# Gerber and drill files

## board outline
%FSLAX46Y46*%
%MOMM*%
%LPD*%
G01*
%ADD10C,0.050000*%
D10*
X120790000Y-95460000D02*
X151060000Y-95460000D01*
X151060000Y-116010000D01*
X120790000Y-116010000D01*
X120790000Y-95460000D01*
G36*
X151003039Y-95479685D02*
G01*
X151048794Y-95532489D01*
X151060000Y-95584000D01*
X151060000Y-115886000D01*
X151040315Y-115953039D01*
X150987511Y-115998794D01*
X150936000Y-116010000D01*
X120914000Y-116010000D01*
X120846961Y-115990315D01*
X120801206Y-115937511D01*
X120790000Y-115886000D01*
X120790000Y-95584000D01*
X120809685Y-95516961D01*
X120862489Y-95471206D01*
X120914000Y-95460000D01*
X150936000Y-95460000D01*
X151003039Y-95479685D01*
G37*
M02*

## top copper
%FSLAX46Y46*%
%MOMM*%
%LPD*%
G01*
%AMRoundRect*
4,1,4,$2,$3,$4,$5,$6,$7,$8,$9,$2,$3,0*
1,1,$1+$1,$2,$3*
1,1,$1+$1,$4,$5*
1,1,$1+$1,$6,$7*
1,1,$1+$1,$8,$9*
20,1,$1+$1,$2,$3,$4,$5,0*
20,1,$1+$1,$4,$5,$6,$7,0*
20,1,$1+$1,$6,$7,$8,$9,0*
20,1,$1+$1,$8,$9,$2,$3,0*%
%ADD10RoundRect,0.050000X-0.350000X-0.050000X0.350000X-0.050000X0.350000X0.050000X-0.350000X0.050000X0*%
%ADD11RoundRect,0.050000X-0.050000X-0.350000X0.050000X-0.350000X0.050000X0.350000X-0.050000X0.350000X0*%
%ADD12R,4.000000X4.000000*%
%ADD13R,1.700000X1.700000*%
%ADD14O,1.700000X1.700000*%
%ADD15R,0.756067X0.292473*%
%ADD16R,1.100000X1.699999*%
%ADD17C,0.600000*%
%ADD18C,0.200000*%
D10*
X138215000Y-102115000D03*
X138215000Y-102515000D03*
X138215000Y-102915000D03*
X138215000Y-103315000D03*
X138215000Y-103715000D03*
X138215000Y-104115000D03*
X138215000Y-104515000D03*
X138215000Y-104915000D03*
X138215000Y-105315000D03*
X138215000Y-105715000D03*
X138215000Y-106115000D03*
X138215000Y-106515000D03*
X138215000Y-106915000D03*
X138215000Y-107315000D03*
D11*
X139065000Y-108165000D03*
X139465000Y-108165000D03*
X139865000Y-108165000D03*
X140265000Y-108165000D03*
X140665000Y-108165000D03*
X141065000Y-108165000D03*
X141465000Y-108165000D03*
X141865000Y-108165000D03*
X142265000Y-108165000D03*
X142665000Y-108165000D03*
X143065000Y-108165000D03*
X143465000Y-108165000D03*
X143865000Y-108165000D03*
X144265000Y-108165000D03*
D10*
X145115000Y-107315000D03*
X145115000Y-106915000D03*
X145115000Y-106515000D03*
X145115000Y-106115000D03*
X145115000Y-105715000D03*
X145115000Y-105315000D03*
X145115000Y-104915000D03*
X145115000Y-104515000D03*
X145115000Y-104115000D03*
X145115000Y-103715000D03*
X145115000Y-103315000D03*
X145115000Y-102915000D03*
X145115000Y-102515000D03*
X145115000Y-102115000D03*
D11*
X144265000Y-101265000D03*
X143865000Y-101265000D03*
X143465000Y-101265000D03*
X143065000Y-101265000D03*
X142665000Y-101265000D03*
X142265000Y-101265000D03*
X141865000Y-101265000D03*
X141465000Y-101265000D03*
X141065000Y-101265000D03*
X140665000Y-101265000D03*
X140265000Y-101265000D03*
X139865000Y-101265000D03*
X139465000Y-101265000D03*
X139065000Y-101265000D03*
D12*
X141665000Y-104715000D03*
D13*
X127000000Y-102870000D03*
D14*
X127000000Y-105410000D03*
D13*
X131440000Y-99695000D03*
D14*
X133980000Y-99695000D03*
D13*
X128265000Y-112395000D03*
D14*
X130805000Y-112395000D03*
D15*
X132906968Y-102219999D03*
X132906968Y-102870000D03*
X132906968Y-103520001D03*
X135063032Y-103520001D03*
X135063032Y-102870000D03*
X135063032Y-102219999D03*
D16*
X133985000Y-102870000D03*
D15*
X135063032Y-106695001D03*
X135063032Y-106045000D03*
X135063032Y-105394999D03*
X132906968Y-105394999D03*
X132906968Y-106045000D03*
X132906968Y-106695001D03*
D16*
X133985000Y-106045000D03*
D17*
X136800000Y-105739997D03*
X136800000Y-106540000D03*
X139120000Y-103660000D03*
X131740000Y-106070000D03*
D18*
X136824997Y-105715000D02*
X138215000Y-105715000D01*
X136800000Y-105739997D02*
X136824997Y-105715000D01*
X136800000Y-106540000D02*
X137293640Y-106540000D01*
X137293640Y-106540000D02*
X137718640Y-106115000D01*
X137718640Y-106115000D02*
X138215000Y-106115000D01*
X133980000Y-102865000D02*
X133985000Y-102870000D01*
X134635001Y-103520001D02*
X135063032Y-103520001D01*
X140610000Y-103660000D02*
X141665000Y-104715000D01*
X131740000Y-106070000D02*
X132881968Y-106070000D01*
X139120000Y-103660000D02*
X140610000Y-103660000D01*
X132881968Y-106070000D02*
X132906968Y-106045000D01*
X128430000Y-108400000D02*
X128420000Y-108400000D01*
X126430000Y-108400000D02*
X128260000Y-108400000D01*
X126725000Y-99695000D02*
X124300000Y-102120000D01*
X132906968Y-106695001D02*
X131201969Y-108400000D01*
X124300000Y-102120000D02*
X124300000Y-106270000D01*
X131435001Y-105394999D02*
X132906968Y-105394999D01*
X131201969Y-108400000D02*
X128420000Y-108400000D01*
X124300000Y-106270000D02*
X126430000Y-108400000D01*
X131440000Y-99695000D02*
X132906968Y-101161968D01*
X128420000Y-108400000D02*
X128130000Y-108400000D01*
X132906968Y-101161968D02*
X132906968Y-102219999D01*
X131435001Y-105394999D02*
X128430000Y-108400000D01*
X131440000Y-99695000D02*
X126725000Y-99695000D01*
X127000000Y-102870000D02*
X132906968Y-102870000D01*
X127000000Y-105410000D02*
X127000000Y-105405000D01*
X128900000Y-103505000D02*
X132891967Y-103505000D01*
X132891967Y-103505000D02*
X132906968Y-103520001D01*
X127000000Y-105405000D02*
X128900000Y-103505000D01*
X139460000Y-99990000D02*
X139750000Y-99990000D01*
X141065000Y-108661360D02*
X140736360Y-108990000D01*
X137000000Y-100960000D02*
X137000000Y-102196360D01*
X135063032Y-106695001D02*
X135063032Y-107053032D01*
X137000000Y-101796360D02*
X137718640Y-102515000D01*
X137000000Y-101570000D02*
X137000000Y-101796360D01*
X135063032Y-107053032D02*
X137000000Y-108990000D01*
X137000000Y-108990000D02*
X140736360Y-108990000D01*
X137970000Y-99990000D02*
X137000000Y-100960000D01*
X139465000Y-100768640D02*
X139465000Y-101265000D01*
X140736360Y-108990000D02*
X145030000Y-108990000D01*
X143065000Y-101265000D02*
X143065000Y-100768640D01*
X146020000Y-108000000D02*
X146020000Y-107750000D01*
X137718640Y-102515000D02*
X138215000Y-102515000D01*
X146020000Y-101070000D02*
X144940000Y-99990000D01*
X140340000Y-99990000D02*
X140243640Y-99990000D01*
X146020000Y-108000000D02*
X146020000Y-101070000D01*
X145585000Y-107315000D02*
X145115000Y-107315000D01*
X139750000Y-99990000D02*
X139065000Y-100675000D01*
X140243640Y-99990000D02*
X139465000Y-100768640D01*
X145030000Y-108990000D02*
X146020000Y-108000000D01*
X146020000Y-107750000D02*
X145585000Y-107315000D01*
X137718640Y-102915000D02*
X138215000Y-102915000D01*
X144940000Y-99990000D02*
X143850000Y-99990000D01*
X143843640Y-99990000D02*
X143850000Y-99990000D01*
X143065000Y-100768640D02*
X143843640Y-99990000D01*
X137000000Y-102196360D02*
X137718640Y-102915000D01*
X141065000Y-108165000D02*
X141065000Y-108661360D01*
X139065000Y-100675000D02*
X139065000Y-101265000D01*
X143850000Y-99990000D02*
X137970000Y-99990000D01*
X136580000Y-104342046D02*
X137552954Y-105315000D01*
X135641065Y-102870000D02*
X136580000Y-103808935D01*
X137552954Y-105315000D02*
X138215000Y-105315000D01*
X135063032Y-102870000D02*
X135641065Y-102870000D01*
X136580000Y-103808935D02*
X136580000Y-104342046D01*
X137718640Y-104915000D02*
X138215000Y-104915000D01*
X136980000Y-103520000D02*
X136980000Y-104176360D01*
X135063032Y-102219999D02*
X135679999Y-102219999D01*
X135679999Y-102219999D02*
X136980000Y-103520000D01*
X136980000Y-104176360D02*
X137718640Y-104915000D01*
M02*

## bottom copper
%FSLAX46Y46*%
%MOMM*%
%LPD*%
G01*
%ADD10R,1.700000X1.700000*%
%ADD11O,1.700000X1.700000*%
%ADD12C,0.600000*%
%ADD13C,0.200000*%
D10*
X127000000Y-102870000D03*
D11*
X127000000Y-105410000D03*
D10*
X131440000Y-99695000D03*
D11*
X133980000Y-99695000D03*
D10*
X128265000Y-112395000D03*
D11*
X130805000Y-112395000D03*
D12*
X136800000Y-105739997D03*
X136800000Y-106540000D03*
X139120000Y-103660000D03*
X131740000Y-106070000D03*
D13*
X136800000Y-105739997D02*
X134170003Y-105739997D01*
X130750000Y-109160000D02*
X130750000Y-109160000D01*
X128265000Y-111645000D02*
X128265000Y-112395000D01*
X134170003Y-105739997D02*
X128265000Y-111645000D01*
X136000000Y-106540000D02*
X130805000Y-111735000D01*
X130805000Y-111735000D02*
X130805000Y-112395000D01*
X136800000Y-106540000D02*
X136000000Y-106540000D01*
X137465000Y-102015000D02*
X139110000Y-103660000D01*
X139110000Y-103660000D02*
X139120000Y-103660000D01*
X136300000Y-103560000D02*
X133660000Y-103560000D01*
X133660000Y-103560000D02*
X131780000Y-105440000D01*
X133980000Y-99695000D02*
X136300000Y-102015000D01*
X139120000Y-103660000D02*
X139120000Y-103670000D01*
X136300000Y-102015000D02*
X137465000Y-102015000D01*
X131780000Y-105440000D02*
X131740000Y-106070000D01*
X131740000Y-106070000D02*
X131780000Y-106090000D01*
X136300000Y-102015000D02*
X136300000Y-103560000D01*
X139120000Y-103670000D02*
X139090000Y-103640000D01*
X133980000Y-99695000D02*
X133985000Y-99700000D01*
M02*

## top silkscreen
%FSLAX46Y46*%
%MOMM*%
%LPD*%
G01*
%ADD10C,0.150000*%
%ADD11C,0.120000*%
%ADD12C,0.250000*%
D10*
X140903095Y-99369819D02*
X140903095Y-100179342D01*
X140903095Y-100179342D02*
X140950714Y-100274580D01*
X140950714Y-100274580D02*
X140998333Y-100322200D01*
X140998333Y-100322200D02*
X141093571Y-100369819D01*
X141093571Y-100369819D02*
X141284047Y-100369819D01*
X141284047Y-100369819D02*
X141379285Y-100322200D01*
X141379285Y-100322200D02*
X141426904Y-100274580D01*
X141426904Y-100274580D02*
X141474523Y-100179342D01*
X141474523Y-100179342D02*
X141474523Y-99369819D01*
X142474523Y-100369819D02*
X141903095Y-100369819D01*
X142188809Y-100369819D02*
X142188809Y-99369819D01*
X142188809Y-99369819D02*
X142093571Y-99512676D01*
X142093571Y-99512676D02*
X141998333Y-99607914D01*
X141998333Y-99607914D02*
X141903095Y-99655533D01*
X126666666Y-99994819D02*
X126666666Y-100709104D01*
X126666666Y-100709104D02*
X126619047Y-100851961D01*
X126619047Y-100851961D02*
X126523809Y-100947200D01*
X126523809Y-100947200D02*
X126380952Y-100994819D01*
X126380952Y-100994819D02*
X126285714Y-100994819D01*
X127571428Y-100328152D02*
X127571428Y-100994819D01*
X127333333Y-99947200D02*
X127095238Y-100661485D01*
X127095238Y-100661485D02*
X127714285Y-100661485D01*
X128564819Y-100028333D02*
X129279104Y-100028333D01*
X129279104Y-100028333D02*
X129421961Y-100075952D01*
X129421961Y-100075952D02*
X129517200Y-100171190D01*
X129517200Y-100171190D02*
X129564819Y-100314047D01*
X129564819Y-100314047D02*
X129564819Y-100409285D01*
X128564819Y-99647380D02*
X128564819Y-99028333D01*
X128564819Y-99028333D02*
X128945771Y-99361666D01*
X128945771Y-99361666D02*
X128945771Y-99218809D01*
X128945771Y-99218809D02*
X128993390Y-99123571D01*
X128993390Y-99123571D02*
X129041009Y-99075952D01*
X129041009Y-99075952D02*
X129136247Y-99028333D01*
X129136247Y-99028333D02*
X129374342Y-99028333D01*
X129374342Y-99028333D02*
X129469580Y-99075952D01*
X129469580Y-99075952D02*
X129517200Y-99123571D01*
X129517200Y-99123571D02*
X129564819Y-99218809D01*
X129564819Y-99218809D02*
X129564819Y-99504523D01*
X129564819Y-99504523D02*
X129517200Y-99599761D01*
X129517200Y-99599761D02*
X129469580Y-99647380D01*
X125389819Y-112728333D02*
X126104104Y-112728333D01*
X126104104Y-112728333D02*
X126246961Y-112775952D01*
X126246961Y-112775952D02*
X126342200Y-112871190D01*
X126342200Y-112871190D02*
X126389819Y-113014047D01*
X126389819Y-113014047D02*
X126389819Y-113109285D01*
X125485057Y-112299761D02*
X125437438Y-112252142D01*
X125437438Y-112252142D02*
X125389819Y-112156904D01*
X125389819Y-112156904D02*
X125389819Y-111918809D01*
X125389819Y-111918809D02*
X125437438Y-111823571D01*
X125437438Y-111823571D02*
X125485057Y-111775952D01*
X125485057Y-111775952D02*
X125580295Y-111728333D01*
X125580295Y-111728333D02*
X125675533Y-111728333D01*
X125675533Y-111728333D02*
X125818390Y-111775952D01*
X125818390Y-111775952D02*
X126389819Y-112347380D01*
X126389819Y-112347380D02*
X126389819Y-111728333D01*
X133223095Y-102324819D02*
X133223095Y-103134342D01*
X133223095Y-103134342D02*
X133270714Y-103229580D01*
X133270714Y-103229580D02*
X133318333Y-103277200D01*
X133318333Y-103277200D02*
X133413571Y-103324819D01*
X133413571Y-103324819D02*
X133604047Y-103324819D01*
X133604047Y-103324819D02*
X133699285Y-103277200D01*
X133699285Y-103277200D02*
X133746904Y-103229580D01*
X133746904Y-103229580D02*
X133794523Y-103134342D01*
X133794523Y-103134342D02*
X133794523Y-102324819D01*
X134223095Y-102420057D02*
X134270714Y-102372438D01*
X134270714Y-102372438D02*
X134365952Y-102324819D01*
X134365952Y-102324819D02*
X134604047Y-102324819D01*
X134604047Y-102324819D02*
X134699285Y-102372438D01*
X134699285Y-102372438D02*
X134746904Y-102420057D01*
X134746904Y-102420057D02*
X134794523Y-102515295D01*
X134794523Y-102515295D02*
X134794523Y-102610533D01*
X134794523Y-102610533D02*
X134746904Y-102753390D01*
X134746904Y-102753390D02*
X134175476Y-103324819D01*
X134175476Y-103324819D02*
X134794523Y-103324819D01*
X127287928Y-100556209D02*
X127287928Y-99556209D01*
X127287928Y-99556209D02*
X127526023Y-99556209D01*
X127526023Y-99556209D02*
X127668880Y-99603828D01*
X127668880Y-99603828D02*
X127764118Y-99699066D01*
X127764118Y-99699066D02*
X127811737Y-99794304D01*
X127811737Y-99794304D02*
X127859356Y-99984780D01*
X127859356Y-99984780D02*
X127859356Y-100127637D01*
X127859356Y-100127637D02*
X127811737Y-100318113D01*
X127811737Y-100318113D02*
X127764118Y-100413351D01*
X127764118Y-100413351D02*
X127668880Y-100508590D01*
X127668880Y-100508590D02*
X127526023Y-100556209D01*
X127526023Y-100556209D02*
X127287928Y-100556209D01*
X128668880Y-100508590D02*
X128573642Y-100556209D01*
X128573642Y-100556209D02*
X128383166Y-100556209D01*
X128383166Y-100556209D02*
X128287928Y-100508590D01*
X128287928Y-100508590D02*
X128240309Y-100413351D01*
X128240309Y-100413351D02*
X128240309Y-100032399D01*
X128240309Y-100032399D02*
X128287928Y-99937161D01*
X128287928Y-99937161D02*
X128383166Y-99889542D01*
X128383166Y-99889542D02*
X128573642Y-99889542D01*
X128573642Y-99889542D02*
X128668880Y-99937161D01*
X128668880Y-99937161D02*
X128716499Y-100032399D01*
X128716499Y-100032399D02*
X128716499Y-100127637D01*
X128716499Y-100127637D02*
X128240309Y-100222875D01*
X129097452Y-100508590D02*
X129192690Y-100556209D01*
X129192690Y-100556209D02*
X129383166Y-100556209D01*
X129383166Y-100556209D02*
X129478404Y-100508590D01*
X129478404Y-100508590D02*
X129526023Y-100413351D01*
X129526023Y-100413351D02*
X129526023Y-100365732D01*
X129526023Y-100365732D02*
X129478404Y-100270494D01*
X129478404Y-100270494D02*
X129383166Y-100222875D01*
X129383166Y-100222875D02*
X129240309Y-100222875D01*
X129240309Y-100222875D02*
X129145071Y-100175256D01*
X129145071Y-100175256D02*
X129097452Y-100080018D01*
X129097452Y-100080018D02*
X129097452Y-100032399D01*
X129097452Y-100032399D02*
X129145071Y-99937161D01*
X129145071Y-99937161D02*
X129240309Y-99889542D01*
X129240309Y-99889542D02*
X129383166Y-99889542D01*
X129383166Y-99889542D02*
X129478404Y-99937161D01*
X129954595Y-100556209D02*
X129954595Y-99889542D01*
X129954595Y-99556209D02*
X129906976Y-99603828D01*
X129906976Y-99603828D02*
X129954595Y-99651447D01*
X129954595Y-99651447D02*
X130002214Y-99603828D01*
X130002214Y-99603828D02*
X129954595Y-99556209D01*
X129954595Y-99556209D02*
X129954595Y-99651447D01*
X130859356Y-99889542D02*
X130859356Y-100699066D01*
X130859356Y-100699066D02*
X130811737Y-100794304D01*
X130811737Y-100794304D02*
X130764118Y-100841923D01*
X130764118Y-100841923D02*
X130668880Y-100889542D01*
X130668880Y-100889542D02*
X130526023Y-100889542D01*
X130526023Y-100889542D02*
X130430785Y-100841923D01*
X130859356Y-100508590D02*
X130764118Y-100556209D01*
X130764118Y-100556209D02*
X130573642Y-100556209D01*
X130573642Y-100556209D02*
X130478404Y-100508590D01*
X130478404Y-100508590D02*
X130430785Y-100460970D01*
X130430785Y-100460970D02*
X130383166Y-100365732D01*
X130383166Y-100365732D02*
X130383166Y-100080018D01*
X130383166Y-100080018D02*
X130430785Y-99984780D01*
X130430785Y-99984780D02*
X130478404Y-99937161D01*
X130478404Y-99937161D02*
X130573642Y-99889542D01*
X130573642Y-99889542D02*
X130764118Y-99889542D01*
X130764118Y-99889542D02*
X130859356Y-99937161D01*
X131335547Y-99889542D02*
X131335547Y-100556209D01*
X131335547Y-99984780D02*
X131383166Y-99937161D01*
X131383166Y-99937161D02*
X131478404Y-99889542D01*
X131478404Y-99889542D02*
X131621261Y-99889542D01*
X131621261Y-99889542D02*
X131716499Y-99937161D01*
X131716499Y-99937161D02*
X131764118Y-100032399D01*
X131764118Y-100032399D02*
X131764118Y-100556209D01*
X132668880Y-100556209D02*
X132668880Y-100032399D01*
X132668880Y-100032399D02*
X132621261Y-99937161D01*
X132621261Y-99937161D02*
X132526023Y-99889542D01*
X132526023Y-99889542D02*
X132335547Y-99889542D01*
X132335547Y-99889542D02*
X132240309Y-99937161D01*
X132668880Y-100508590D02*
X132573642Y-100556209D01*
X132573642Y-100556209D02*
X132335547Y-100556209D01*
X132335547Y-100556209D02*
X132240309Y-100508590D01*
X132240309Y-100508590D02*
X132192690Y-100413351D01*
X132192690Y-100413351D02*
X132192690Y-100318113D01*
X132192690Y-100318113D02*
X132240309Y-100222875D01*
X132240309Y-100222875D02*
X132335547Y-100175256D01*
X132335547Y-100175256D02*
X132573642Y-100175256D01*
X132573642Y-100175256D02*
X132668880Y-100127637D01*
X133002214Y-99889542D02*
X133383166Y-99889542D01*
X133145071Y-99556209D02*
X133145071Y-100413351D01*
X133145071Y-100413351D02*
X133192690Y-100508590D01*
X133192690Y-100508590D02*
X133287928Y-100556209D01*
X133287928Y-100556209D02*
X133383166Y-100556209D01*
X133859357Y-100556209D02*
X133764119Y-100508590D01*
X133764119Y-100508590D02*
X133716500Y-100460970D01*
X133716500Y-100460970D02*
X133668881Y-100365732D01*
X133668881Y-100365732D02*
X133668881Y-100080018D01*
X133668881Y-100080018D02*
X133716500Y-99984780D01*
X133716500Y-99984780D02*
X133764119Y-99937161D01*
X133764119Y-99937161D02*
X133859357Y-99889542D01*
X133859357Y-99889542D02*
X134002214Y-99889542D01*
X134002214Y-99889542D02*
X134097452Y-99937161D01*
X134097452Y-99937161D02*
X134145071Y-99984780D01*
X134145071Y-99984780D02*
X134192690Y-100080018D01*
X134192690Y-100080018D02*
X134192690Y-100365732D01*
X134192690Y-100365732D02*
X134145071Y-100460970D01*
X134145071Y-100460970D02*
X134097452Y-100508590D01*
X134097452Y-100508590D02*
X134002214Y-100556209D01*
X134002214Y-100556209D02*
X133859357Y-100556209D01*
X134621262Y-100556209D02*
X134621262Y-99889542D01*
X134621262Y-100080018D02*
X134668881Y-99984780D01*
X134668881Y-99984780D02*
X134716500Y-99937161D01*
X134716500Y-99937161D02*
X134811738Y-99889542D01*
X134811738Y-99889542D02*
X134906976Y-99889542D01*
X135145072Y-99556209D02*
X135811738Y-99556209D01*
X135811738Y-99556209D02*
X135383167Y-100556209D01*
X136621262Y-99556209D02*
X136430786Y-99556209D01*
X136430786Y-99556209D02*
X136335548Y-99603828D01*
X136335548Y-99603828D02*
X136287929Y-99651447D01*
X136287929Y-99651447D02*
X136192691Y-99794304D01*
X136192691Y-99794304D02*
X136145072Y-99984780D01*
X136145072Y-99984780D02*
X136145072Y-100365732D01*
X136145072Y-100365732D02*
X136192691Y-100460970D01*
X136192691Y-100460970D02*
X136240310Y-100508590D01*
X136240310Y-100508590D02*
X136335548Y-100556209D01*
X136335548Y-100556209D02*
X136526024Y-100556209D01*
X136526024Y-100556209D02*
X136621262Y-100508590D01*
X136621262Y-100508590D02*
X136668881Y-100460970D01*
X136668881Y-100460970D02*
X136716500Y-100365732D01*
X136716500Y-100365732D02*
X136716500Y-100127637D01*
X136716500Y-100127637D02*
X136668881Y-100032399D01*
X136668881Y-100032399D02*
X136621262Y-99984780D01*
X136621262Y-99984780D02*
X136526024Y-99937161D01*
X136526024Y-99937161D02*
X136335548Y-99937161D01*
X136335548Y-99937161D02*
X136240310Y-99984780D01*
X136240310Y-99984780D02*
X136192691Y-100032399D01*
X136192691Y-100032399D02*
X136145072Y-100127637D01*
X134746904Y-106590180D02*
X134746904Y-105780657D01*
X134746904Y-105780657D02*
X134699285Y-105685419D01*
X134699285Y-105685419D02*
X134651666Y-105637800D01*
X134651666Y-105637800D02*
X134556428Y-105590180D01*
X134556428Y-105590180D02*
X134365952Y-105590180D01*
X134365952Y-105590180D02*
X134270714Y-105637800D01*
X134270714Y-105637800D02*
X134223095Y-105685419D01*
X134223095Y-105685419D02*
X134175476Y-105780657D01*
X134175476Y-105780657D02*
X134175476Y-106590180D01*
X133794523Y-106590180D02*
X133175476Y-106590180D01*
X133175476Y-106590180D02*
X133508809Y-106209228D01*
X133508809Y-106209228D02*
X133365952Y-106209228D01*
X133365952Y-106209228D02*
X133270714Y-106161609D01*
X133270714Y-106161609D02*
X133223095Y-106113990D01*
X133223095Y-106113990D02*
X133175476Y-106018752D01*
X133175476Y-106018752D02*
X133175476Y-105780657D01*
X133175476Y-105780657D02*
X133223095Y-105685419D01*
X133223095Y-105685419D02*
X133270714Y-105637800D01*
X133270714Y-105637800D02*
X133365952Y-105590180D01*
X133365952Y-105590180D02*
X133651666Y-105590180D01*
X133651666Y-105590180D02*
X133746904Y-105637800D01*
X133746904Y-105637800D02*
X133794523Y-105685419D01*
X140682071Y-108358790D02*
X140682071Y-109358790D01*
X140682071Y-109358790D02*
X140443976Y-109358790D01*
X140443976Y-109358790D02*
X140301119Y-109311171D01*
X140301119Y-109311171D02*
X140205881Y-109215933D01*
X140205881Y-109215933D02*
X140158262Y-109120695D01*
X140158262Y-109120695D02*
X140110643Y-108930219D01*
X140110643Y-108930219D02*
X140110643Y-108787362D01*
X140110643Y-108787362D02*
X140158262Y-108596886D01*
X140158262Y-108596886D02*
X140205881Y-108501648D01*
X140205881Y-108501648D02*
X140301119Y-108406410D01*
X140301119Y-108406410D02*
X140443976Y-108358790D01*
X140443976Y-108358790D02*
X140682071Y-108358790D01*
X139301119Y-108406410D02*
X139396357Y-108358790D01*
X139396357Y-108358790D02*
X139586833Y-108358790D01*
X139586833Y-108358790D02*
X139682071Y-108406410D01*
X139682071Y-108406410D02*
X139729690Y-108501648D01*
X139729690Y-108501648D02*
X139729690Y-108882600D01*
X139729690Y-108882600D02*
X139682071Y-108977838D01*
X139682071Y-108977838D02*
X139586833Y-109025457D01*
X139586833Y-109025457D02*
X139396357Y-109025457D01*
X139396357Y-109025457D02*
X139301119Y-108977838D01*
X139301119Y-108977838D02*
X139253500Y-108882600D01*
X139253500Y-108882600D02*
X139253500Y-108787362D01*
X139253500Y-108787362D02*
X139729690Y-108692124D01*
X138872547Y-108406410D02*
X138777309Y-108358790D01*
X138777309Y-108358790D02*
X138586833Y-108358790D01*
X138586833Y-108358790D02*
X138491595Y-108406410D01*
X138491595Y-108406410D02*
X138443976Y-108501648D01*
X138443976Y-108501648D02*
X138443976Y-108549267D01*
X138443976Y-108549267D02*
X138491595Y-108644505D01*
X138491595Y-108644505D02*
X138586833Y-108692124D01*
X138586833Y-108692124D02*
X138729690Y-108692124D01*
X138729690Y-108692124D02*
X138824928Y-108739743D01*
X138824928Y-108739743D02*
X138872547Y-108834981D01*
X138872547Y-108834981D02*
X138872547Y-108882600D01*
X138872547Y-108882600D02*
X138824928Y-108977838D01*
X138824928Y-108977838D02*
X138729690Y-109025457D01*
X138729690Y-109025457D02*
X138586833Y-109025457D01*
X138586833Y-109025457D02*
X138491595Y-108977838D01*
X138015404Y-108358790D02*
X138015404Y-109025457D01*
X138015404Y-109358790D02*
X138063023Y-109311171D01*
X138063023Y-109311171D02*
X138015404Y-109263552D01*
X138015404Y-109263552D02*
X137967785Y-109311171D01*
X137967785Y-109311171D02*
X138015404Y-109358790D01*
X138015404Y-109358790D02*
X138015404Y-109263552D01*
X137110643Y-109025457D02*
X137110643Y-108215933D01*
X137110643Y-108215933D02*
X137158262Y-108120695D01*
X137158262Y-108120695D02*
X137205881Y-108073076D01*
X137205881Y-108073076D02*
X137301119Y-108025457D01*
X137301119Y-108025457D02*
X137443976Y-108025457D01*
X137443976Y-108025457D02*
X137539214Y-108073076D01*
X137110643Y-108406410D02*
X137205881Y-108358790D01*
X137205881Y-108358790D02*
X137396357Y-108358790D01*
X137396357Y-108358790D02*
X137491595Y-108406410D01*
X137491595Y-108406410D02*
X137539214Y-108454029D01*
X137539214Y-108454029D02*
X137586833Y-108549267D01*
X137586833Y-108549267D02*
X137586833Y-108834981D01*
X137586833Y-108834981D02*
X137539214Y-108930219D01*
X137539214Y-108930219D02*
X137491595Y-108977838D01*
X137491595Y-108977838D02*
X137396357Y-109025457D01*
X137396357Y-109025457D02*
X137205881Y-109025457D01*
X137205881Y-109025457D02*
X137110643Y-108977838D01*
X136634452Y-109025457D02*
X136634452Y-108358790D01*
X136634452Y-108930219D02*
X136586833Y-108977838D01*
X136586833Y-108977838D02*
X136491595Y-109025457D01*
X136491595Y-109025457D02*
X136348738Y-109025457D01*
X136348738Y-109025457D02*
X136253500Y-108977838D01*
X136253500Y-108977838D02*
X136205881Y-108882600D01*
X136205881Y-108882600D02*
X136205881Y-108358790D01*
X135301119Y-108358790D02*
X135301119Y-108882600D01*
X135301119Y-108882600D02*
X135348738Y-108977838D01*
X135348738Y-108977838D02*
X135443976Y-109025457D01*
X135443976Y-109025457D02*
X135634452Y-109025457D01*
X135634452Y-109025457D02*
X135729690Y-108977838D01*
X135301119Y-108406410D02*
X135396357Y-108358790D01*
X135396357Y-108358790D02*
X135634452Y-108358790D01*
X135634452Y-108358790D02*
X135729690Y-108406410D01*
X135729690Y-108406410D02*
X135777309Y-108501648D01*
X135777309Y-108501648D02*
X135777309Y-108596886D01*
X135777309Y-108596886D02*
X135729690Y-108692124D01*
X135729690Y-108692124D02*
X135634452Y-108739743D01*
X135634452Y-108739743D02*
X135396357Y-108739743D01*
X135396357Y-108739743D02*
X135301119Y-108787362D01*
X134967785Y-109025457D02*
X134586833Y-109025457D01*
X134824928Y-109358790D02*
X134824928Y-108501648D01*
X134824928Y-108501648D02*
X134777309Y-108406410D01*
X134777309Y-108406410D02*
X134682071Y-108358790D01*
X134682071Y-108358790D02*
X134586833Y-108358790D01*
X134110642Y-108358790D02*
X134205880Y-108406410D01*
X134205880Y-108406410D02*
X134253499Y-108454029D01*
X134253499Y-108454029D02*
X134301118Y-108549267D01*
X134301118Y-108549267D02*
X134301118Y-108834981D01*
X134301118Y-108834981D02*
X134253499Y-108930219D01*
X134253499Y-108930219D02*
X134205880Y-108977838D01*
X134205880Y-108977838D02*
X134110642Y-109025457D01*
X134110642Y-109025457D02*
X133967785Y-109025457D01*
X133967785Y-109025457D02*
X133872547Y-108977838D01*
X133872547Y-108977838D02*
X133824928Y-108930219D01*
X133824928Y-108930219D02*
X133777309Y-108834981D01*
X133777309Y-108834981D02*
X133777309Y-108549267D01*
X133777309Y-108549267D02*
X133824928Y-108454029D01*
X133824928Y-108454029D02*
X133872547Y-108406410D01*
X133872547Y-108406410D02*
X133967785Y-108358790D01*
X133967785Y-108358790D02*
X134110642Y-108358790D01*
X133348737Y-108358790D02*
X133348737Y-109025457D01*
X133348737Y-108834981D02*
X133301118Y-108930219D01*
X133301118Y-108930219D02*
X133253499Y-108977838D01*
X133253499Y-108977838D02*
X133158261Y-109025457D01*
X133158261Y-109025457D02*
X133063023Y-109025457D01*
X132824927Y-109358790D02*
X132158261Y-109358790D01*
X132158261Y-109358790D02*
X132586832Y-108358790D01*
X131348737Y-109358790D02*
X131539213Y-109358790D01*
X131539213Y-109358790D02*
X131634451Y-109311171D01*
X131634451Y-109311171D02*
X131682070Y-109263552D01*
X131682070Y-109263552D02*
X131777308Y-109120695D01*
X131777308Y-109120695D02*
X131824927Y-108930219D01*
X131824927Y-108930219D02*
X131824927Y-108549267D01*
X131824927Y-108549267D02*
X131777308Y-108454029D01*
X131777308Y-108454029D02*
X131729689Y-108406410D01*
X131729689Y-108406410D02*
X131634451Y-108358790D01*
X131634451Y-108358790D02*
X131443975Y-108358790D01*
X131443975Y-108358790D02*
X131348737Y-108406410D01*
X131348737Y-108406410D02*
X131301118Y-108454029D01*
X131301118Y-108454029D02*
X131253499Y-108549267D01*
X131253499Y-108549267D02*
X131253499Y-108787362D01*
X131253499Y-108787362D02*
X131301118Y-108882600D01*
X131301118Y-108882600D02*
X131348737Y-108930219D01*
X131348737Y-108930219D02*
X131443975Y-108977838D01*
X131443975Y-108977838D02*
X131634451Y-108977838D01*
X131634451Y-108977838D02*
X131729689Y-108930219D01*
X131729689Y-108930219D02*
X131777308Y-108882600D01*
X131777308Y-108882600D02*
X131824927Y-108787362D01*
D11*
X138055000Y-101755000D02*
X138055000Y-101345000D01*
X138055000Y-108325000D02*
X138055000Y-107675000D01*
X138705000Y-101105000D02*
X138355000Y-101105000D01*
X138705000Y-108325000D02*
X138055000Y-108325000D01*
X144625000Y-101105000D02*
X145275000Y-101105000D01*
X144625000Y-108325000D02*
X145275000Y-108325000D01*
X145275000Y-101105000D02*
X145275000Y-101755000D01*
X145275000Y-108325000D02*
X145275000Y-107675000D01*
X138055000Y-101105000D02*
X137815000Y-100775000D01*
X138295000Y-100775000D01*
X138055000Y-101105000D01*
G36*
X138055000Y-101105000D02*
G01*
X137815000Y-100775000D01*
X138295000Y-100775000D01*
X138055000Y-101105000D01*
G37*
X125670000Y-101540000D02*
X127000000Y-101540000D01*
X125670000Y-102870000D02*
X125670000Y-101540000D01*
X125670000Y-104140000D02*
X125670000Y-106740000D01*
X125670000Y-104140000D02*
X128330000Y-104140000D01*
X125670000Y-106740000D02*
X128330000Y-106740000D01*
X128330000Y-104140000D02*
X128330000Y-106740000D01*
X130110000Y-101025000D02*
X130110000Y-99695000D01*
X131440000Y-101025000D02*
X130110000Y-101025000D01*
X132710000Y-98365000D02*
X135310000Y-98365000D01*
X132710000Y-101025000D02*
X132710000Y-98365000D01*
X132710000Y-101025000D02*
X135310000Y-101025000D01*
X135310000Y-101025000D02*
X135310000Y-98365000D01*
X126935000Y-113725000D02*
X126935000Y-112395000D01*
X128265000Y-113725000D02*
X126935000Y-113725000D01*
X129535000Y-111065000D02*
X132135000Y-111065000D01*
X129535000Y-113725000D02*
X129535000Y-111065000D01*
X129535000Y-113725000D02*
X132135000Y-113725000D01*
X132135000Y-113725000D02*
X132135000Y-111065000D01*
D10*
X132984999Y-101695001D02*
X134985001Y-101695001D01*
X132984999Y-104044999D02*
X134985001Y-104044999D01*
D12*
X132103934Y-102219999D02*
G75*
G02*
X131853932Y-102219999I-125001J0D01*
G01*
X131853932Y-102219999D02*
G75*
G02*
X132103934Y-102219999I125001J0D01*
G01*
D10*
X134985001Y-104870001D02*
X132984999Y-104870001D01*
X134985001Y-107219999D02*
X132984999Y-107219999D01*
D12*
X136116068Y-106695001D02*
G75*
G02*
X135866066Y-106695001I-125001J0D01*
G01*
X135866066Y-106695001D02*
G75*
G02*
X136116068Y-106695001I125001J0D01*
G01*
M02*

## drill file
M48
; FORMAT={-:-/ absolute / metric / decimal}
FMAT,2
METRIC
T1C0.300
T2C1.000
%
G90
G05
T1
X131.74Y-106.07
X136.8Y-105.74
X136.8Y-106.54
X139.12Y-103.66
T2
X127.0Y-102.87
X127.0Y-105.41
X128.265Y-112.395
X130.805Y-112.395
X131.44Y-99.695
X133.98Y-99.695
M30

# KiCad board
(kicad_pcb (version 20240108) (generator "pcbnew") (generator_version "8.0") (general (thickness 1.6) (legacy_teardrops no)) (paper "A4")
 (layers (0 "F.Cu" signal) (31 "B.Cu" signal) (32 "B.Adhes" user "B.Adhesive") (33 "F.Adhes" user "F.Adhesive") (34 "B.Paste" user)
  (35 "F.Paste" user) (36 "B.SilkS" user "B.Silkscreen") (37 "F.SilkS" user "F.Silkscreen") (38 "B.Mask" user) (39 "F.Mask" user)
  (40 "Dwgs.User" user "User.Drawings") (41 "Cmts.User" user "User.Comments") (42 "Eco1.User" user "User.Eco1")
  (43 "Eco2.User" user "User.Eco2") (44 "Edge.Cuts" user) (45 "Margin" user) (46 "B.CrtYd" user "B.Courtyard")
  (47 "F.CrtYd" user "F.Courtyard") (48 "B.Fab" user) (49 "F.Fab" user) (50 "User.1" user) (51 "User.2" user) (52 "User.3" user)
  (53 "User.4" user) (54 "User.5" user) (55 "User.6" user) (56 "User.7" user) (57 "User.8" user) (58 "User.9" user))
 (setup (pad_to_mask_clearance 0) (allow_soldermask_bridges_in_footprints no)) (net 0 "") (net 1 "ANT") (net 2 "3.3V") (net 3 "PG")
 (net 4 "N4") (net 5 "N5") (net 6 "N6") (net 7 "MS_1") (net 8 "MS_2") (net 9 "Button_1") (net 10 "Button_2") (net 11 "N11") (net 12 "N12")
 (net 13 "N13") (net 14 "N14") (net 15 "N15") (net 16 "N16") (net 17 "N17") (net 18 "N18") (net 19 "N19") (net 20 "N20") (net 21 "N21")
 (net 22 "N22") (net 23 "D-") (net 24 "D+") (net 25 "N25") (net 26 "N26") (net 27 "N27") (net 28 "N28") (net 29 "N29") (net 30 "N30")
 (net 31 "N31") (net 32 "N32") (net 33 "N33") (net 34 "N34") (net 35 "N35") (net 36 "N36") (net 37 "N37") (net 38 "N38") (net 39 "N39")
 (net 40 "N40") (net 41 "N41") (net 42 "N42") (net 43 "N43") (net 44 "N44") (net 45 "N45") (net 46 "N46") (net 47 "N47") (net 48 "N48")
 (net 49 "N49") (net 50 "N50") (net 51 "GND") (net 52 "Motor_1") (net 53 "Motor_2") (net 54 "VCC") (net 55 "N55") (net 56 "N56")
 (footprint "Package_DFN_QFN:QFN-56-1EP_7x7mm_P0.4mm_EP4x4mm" (layer "F.Cu") (at 141.665 104.715)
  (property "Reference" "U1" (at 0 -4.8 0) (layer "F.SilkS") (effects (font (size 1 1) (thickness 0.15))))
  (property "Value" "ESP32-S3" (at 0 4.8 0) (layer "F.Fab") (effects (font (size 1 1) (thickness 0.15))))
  (fp_line (start -3.61 -2.96) (end -3.61 -3.37) (stroke (width 0.12) (type solid)) (layer "F.SilkS"))
  (fp_line (start -3.61 3.61) (end -3.61 2.96) (stroke (width 0.12) (type solid)) (layer "F.SilkS"))
  (fp_line (start -2.96 -3.61) (end -3.31 -3.61) (stroke (width 0.12) (type solid)) (layer "F.SilkS"))
  (fp_line (start -2.96 3.61) (end -3.61 3.61) (stroke (width 0.12) (type solid)) (layer "F.SilkS"))
  (fp_line (start 2.96 -3.61) (end 3.61 -3.61) (stroke (width 0.12) (type solid)) (layer "F.SilkS"))
  (fp_line (start 2.96 3.61) (end 3.61 3.61) (stroke (width 0.12) (type solid)) (layer "F.SilkS"))
  (fp_line (start 3.61 -3.61) (end 3.61 -2.96) (stroke (width 0.12) (type solid)) (layer "F.SilkS"))
  (fp_line (start 3.61 3.61) (end 3.61 2.96) (stroke (width 0.12) (type solid)) (layer "F.SilkS"))
  (fp_poly
   (pts (xy -3.61 -3.61) (xy -3.85 -3.94) (xy -3.37 -3.94) (xy -3.61 -3.61)) (stroke (width 0.12) (type solid)) (fill solid)
   (layer "F.SilkS"))
  (pad "" smd roundrect (at -1.33 -1.33) (size 1.07 1.07) (layers "F.Paste") (roundrect_rratio 0.233645))
  (pad "" smd roundrect (at -1.33 0) (size 1.07 1.07) (layers "F.Paste") (roundrect_rratio 0.233645))
  (pad "" smd roundrect (at -1.33 1.33) (size 1.07 1.07) (layers "F.Paste") (roundrect_rratio 0.233645))
  (pad "" smd roundrect (at 0 -1.33) (size 1.07 1.07) (layers "F.Paste") (roundrect_rratio 0.233645))
  (pad "" smd roundrect (at 0 0) (size 1.07 1.07) (layers "F.Paste") (roundrect_rratio 0.233645))
  (pad "" smd roundrect (at 0 1.33) (size 1.07 1.07) (layers "F.Paste") (roundrect_rratio 0.233645))
  (pad "" smd roundrect (at 1.33 -1.33) (size 1.07 1.07) (layers "F.Paste") (roundrect_rratio 0.233645))
  (pad "" smd roundrect (at 1.33 0) (size 1.07 1.07) (layers "F.Paste") (roundrect_rratio 0.233645))
  (pad "" smd roundrect (at 1.33 1.33) (size 1.07 1.07) (layers "F.Paste") (roundrect_rratio 0.233645))
  (pad "1" smd roundrect (at -3.45 -2.6) (size 0.8 0.2) (layers "F.Cu" "F.Paste" "F.Mask") (roundrect_rratio 0.25) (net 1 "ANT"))
  (pad "2" smd roundrect (at -3.45 -2.2) (size 0.8 0.2) (layers "F.Cu" "F.Paste" "F.Mask") (roundrect_rratio 0.25) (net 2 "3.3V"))
  (pad "3" smd roundrect (at -3.45 -1.8) (size 0.8 0.2) (layers "F.Cu" "F.Paste" "F.Mask") (roundrect_rratio 0.25) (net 2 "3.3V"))
  (pad "4" smd roundrect (at -3.45 -1.4) (size 0.8 0.2) (layers "F.Cu" "F.Paste" "F.Mask") (roundrect_rratio 0.25) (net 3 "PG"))
  (pad "5" smd roundrect (at -3.45 -1) (size 0.8 0.2) (layers "F.Cu" "F.Paste" "F.Mask") (roundrect_rratio 0.25) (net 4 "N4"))
  (pad "6" smd roundrect (at -3.45 -0.6) (size 0.8 0.2) (layers "F.Cu" "F.Paste" "F.Mask") (roundrect_rratio 0.25) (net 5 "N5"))
  (pad "7" smd roundrect (at -3.45 -0.2) (size 0.8 0.2) (layers "F.Cu" "F.Paste" "F.Mask") (roundrect_rratio 0.25) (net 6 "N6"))
  (pad "8" smd roundrect (at -3.45 0.2) (size 0.8 0.2) (layers "F.Cu" "F.Paste" "F.Mask") (roundrect_rratio 0.25) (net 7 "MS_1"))
  (pad "9" smd roundrect (at -3.45 0.6) (size 0.8 0.2) (layers "F.Cu" "F.Paste" "F.Mask") (roundrect_rratio 0.25) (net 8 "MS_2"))
  (pad "10" smd roundrect (at -3.45 1) (size 0.8 0.2) (layers "F.Cu" "F.Paste" "F.Mask") (roundrect_rratio 0.25) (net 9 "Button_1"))
  (pad "11" smd roundrect (at -3.45 1.4) (size 0.8 0.2) (layers "F.Cu" "F.Paste" "F.Mask") (roundrect_rratio 0.25) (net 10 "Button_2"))
  (pad "12" smd roundrect (at -3.45 1.8) (size 0.8 0.2) (layers "F.Cu" "F.Paste" "F.Mask") (roundrect_rratio 0.25) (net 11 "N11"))
  (pad "13" smd roundrect (at -3.45 2.2) (size 0.8 0.2) (layers "F.Cu" "F.Paste" "F.Mask") (roundrect_rratio 0.25) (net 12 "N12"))
  (pad "14" smd roundrect (at -3.45 2.6) (size 0.8 0.2) (layers "F.Cu" "F.Paste" "F.Mask") (roundrect_rratio 0.25) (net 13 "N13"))
  (pad "15" smd roundrect (at -2.6 3.45) (size 0.2 0.8) (layers "F.Cu" "F.Paste" "F.Mask") (roundrect_rratio 0.25) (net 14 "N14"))
  (pad "16" smd roundrect (at -2.2 3.45) (size 0.2 0.8) (layers "F.Cu" "F.Paste" "F.Mask") (roundrect_rratio 0.25) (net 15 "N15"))
  (pad "17" smd roundrect (at -1.8 3.45) (size 0.2 0.8) (layers "F.Cu" "F.Paste" "F.Mask") (roundrect_rratio 0.25) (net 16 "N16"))
  (pad "18" smd roundrect (at -1.4 3.45) (size 0.2 0.8) (layers "F.Cu" "F.Paste" "F.Mask") (roundrect_rratio 0.25) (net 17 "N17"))
  (pad "19" smd roundrect (at -1 3.45) (size 0.2 0.8) (layers "F.Cu" "F.Paste" "F.Mask") (roundrect_rratio 0.25) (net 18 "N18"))
  (pad "20" smd roundrect (at -0.6 3.45) (size 0.2 0.8) (layers "F.Cu" "F.Paste" "F.Mask") (roundrect_rratio 0.25) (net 2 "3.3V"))
  (pad "21" smd roundrect (at -0.2 3.45) (size 0.2 0.8) (layers "F.Cu" "F.Paste" "F.Mask") (roundrect_rratio 0.25) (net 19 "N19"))
  (pad "22" smd roundrect (at 0.2 3.45) (size 0.2 0.8) (layers "F.Cu" "F.Paste" "F.Mask") (roundrect_rratio 0.25) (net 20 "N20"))
  (pad "23" smd roundrect (at 0.6 3.45) (size 0.2 0.8) (layers "F.Cu" "F.Paste" "F.Mask") (roundrect_rratio 0.25) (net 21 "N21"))
  (pad "24" smd roundrect (at 1 3.45) (size 0.2 0.8) (layers "F.Cu" "F.Paste" "F.Mask") (roundrect_rratio 0.25) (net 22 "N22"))
  (pad "25" smd roundrect (at 1.4 3.45) (size 0.2 0.8) (layers "F.Cu" "F.Paste" "F.Mask") (roundrect_rratio 0.25) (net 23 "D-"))
  (pad "26" smd roundrect (at 1.8 3.45) (size 0.2 0.8) (layers "F.Cu" "F.Paste" "F.Mask") (roundrect_rratio 0.25) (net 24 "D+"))
  (pad "27" smd roundrect (at 2.2 3.45) (size 0.2 0.8) (layers "F.Cu" "F.Paste" "F.Mask") (roundrect_rratio 0.25) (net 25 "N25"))
  (pad "28" smd roundrect (at 2.6 3.45) (size 0.2 0.8) (layers "F.Cu" "F.Paste" "F.Mask") (roundrect_rratio 0.25) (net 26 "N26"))
  (pad "29" smd roundrect (at 3.45 2.6) (size 0.8 0.2) (layers "F.Cu" "F.Paste" "F.Mask") (roundrect_rratio 0.25) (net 2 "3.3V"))
  (pad "30" smd roundrect (at 3.45 2.2) (size 0.8 0.2) (layers "F.Cu" "F.Paste" "F.Mask") (roundrect_rratio 0.25) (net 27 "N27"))
  (pad "31" smd roundrect (at 3.45 1.8) (size 0.8 0.2) (layers "F.Cu" "F.Paste" "F.Mask") (roundrect_rratio 0.25) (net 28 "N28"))
  (pad "32" smd roundrect (at 3.45 1.4) (size 0.8 0.2) (layers "F.Cu" "F.Paste" "F.Mask") (roundrect_rratio 0.25) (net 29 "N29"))
  (pad "33" smd roundrect (at 3.45 1) (size 0.8 0.2) (layers "F.Cu" "F.Paste" "F.Mask") (roundrect_rratio 0.25) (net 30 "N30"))
  (pad "34" smd roundrect (at 3.45 0.6) (size 0.8 0.2) (layers "F.Cu" "F.Paste" "F.Mask") (roundrect_rratio 0.25) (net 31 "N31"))
  (pad "35" smd roundrect (at 3.45 0.2) (size 0.8 0.2) (layers "F.Cu" "F.Paste" "F.Mask") (roundrect_rratio 0.25) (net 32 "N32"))
  (pad "36" smd roundrect (at 3.45 -0.2) (size 0.8 0.2) (layers "F.Cu" "F.Paste" "F.Mask") (roundrect_rratio 0.25) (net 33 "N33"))
  (pad "37" smd roundrect (at 3.45 -0.6) (size 0.8 0.2) (layers "F.Cu" "F.Paste" "F.Mask") (roundrect_rratio 0.25) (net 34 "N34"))
  (pad "38" smd roundrect (at 3.45 -1) (size 0.8 0.2) (layers "F.Cu" "F.Paste" "F.Mask") (roundrect_rratio 0.25) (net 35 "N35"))
  (pad "39" smd roundrect (at 3.45 -1.4) (size 0.8 0.2) (layers "F.Cu" "F.Paste" "F.Mask") (roundrect_rratio 0.25) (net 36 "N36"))
  (pad "40" smd roundrect (at 3.45 -1.8) (size 0.8 0.2) (layers "F.Cu" "F.Paste" "F.Mask") (roundrect_rratio 0.25) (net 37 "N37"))
  (pad "41" smd roundrect (at 3.45 -2.2) (size 0.8 0.2) (layers "F.Cu" "F.Paste" "F.Mask") (roundrect_rratio 0.25) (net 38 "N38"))
  (pad "42" smd roundrect (at 3.45 -2.6) (size 0.8 0.2) (layers "F.Cu" "F.Paste" "F.Mask") (roundrect_rratio 0.25) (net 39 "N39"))
  (pad "43" smd roundrect (at 2.6 -3.45) (size 0.2 0.8) (layers "F.Cu" "F.Paste" "F.Mask") (roundrect_rratio 0.25) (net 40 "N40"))
  (pad "44" smd roundrect (at 2.2 -3.45) (size 0.2 0.8) (layers "F.Cu" "F.Paste" "F.Mask") (roundrect_rratio 0.25) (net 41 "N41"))
  (pad "45" smd roundrect (at 1.8 -3.45) (size 0.2 0.8) (layers "F.Cu" "F.Paste" "F.Mask") (roundrect_rratio 0.25) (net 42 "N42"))
  (pad "46" smd roundrect (at 1.4 -3.45) (size 0.2 0.8) (layers "F.Cu" "F.Paste" "F.Mask") (roundrect_rratio 0.25) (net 2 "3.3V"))
  (pad "47" smd roundrect (at 1 -3.45) (size 0.2 0.8) (layers "F.Cu" "F.Paste" "F.Mask") (roundrect_rratio 0.25) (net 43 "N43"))
  (pad "48" smd roundrect (at 0.6 -3.45) (size 0.2 0.8) (layers "F.Cu" "F.Paste" "F.Mask") (roundrect_rratio 0.25) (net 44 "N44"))
  (pad "49" smd roundrect (at 0.2 -3.45) (size 0.2 0.8) (layers "F.Cu" "F.Paste" "F.Mask") (roundrect_rratio 0.25) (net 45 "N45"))
  (pad "50" smd roundrect (at -0.2 -3.45) (size 0.2 0.8) (layers "F.Cu" "F.Paste" "F.Mask") (roundrect_rratio 0.25) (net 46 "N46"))
  (pad "51" smd roundrect (at -0.6 -3.45) (size 0.2 0.8) (layers "F.Cu" "F.Paste" "F.Mask") (roundrect_rratio 0.25) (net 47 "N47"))
  (pad "52" smd roundrect (at -1 -3.45) (size 0.2 0.8) (layers "F.Cu" "F.Paste" "F.Mask") (roundrect_rratio 0.25) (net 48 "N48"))
  (pad "53" smd roundrect (at -1.4 -3.45) (size 0.2 0.8) (layers "F.Cu" "F.Paste" "F.Mask") (roundrect_rratio 0.25) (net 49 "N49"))
  (pad "54" smd roundrect (at -1.8 -3.45) (size 0.2 0.8) (layers "F.Cu" "F.Paste" "F.Mask") (roundrect_rratio 0.25) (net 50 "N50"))
  (pad "55" smd roundrect (at -2.2 -3.45) (size 0.2 0.8) (layers "F.Cu" "F.Paste" "F.Mask") (roundrect_rratio 0.25) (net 2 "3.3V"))
  (pad "56" smd roundrect (at -2.6 -3.45) (size 0.2 0.8) (layers "F.Cu" "F.Paste" "F.Mask") (roundrect_rratio 0.25) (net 2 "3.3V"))
  (pad "57" smd rect (at 0 0) (size 4 4) (layers "F.Cu" "F.Mask") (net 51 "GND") (zone_connect 2)))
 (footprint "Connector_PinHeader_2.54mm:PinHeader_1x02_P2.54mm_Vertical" (layer "F.Cu") (at 127 102.87)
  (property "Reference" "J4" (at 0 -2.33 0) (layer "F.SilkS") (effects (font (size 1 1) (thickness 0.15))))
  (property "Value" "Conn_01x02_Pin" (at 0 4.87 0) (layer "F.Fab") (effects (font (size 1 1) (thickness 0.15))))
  (fp_line (start -1.33 -1.33) (end 0 -1.33) (stroke (width 0.12) (type solid)) (layer "F.SilkS"))
  (fp_line (start -1.33 0) (end -1.33 -1.33) (stroke (width 0.12) (type solid)) (layer "F.SilkS"))
  (fp_line (start -1.33 1.27) (end -1.33 3.87) (stroke (width 0.12) (type solid)) (layer "F.SilkS"))
  (fp_line (start -1.33 1.27) (end 1.33 1.27) (stroke (width 0.12) (type solid)) (layer "F.SilkS"))
  (fp_line (start -1.33 3.87) (end 1.33 3.87) (stroke (width 0.12) (type solid)) (layer "F.SilkS"))
  (fp_line (start 1.33 1.27) (end 1.33 3.87) (stroke (width 0.12) (type solid)) (layer "F.SilkS"))
  (pad "1" thru_hole rect (at 0 0) (size 1.7 1.7) (drill 1) (layers "*.Cu" "*.Mask") (remove_unused_layers no) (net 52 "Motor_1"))
  (pad "2" thru_hole oval (at 0 2.54) (size 1.7 1.7) (drill 1) (layers "*.Cu" "*.Mask") (remove_unused_layers no) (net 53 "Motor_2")))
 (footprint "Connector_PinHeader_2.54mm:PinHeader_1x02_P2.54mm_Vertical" (layer "F.Cu") (at 131.44 99.695 90)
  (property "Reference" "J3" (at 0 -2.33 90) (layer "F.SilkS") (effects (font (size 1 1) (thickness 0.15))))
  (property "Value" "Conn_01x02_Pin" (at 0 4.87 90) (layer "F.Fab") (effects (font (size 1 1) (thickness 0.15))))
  (fp_line (start -1.33 -1.33) (end 0 -1.33) (stroke (width 0.12) (type solid)) (layer "F.SilkS"))
  (fp_line (start -1.33 0) (end -1.33 -1.33) (stroke (width 0.12) (type solid)) (layer "F.SilkS"))
  (fp_line (start 1.33 1.27) (end 1.33 3.87) (stroke (width 0.12) (type solid)) (layer "F.SilkS"))
  (fp_line (start -1.33 1.27) (end 1.33 1.27) (stroke (width 0.12) (type solid)) (layer "F.SilkS"))
  (fp_line (start -1.33 1.27) (end -1.33 3.87) (stroke (width 0.12) (type solid)) (layer "F.SilkS"))
  (fp_line (start -1.33 3.87) (end 1.33 3.87) (stroke (width 0.12) (type solid)) (layer "F.SilkS"))
  (pad "1" thru_hole rect (at 0 0 90) (size 1.7 1.7) (drill 1) (layers "*.Cu" "*.Mask") (remove_unused_layers no) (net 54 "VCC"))
  (pad "2" thru_hole oval (at 0 2.54 90) (size 1.7 1.7) (drill 1) (layers "*.Cu" "*.Mask") (remove_unused_layers no) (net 51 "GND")))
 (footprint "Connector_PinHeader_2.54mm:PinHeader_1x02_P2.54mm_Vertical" (layer "F.Cu") (at 128.265 112.395 90)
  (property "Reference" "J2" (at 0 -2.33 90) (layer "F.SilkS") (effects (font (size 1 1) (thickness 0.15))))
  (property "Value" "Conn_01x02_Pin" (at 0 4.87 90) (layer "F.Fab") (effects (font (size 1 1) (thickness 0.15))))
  (fp_line (start -1.33 -1.33) (end 0 -1.33) (stroke (width 0.12) (type solid)) (layer "F.SilkS"))
  (fp_line (start -1.33 0) (end -1.33 -1.33) (stroke (width 0.12) (type solid)) (layer "F.SilkS"))
  (fp_line (start 1.33 1.27) (end 1.33 3.87) (stroke (width 0.12) (type solid)) (layer "F.SilkS"))
  (fp_line (start -1.33 1.27) (end 1.33 1.27) (stroke (width 0.12) (type solid)) (layer "F.SilkS"))
  (fp_line (start -1.33 1.27) (end -1.33 3.87) (stroke (width 0.12) (type solid)) (layer "F.SilkS"))
  (fp_line (start -1.33 3.87) (end 1.33 3.87) (stroke (width 0.12) (type solid)) (layer "F.SilkS"))
  (pad "1" thru_hole rect (at 0 0 90) (size 1.7 1.7) (drill 1) (layers "*.Cu" "*.Mask") (remove_unused_layers no) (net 9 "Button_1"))
  (pad "2" thru_hole oval (at 0 2.54 90) (size 1.7 1.7) (drill 1) (layers "*.Cu" "*.Mask") (remove_unused_layers no) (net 10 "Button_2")))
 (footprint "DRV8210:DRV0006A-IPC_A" (layer "F.Cu") (at 133.985 102.87)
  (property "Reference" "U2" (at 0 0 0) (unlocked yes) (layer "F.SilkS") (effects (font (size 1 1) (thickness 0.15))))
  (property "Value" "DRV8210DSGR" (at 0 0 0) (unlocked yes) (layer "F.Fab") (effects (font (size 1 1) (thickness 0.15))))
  (fp_line (start -1.000001 -1.174999) (end 1.000001 -1.174999) (stroke (width 0.15) (type solid)) (layer "F.SilkS"))
  (fp_line (start -1.000001 1.174999) (end 1.000001 1.174999) (stroke (width 0.15) (type solid)) (layer "F.SilkS"))
  (fp_circle (center -2.006067 -0.650001) (end -1.881066 -0.650001) (stroke (width 0.25) (type solid)) (fill none) (layer "F.SilkS"))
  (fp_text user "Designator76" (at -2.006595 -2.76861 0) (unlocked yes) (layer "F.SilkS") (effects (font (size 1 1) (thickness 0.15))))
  (pad "1" smd rect (at -1.078032 -0.650001) (size 0.756067 0.292473) (layers "F.Cu" "F.Paste" "F.Mask") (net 54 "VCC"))
  (pad "2" smd rect (at -1.078032 0) (size 0.756067 0.292473) (layers "F.Cu" "F.Paste" "F.Mask") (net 52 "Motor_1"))
  (pad "3" smd rect (at -1.078032 0.650001) (size 0.756067 0.292473) (layers "F.Cu" "F.Paste" "F.Mask") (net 53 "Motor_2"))
  (pad "4" smd rect (at 1.078032 0.650001) (size 0.756067 0.292473) (layers "F.Cu" "F.Paste" "F.Mask") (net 51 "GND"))
  (pad "5" smd rect (at 1.078032 0) (size 0.756067 0.292473) (layers "F.Cu" "F.Paste" "F.Mask") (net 8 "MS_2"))
  (pad "6" smd rect (at 1.078032 -0.650001) (size 0.756067 0.292473) (layers "F.Cu" "F.Paste" "F.Mask") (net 7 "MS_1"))
  (pad "7" smd rect (at 0 0) (size 1.1 1.699999) (layers "F.Cu" "F.Mask") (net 51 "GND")))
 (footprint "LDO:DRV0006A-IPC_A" (layer "F.Cu") (at 133.985 106.045 180)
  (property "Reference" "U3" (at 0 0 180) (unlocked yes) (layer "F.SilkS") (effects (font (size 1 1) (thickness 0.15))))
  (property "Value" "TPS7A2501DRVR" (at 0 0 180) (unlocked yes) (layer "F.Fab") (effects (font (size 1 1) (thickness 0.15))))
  (fp_line (start -1.000001 1.174999) (end 1.000001 1.174999) (stroke (width 0.15) (type solid)) (layer "F.SilkS"))
  (fp_line (start -1.000001 -1.174999) (end 1.000001 -1.174999) (stroke (width 0.15) (type solid)) (layer "F.SilkS"))
  (fp_circle (center -2.006067 -0.650001) (end -1.881066 -0.650001) (stroke (width 0.25) (type solid)) (fill none) (layer "F.SilkS"))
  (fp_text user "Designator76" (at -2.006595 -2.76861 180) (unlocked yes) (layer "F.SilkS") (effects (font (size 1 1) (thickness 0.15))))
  (pad "1" smd rect (at -1.078032 -0.650001 180) (size 0.756067 0.292473) (layers "F.Cu" "F.Paste" "F.Mask") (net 2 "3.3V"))
  (pad "2" smd rect (at -1.078032 0 180) (size 0.756067 0.292473) (layers "F.Cu" "F.Paste" "F.Mask") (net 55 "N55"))
  (pad "3" smd rect (at -1.078032 0.650001 180) (size 0.756067 0.292473) (layers "F.Cu" "F.Paste" "F.Mask") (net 3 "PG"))
  (pad "4" smd rect (at 1.078032 0.650001 180) (size 0.756067 0.292473) (layers "F.Cu" "F.Paste" "F.Mask") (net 54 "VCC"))
  (pad "5" smd rect (at 1.078032 0 180) (size 0.756067 0.292473) (layers "F.Cu" "F.Paste" "F.Mask") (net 51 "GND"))
  (pad "6" smd rect (at 1.078032 -0.650001 180) (size 0.756067 0.292473) (layers "F.Cu" "F.Paste" "F.Mask") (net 54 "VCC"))
  (pad "7" smd rect (at 0 0 180) (size 1.1 1.699999) (layers "F.Cu" "F.Mask") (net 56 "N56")))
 (gr_rect (start 120.79 95.46) (end 151.06 116.01) (stroke (width 0.05) (type default)) (fill none) (layer "Edge.Cuts"))
 (segment (start 136.824997 105.715) (end 138.215 105.715) (width 0.2) (layer "F.Cu") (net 9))
 (segment (start 136.8 105.739997) (end 136.824997 105.715) (width 0.2) (layer "F.Cu") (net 9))
 (via (at 136.8 105.739997) (size 0.6) (drill 0.3) (layers "F.Cu" "B.Cu") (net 9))
 (segment (start 136.8 105.739997) (end 134.170003 105.739997) (width 0.2) (layer "B.Cu") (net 9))
 (segment (start 130.75 109.16) (end 130.75 109.16) (width 0.2) (layer "B.Cu") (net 9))
 (segment (start 128.265 111.645) (end 128.265 112.395) (width 0.2) (layer "B.Cu") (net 9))
 (segment (start 134.170003 105.739997) (end 128.265 111.645) (width 0.2) (layer "B.Cu") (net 9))
 (segment (start 136.8 106.54) (end 137.29364 106.54) (width 0.2) (layer "F.Cu") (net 10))
 (segment (start 137.29364 106.54) (end 137.71864 106.115) (width 0.2) (layer "F.Cu") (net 10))
 (segment (start 137.71864 106.115) (end 138.215 106.115) (width 0.2) (layer "F.Cu") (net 10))
 (via (at 136.8 106.54) (size 0.6) (drill 0.3) (layers "F.Cu" "B.Cu") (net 10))
 (segment (start 136 106.54) (end 130.805 111.735) (width 0.2) (layer "B.Cu") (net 10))
 (segment (start 130.805 111.735) (end 130.805 112.395) (width 0.2) (layer "B.Cu") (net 10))
 (segment (start 136.8 106.54) (end 136 106.54) (width 0.2) (layer "B.Cu") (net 10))
 (segment (start 133.98 102.865) (end 133.985 102.87) (width 0.2) (layer "F.Cu") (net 51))
 (segment (start 134.635001 103.520001) (end 135.063032 103.520001) (width 0.2) (layer "F.Cu") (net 51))
 (segment (start 140.61 103.66) (end 141.665 104.715) (width 0.2) (layer "F.Cu") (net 51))
 (segment (start 131.74 106.07) (end 132.881968 106.07) (width 0.2) (layer "F.Cu") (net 51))
 (segment (start 139.12 103.66) (end 140.61 103.66) (width 0.2) (layer "F.Cu") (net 51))
 (segment (start 132.881968 106.07) (end 132.906968 106.045) (width 0.2) (layer "F.Cu") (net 51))
 (via (at 139.12 103.66) (size 0.6) (drill 0.3) (layers "F.Cu" "B.Cu") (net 51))
 (via (at 131.74 106.07) (size 0.6) (drill 0.3) (layers "F.Cu" "B.Cu") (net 51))
 (segment (start 137.465 102.015) (end 139.11 103.66) (width 0.2) (layer "B.Cu") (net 51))
 (segment (start 139.11 103.66) (end 139.12 103.66) (width 0.2) (layer "B.Cu") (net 51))
 (segment (start 136.3 103.56) (end 133.66 103.56) (width 0.2) (layer "B.Cu") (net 51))
 (segment (start 133.66 103.56) (end 131.78 105.44) (width 0.2) (layer "B.Cu") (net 51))
 (segment (start 133.98 99.695) (end 136.3 102.015) (width 0.2) (layer "B.Cu") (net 51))
 (segment (start 139.12 103.66) (end 139.12 103.67) (width 0.2) (layer "B.Cu") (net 51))
 (segment (start 136.3 102.015) (end 137.465 102.015) (width 0.2) (layer "B.Cu") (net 51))
 (segment (start 131.78 105.44) (end 131.74 106.07) (width 0.2) (layer "B.Cu") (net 51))
 (segment (start 131.74 106.07) (end 131.78 106.09) (width 0.2) (layer "B.Cu") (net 51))
 (segment (start 136.3 102.015) (end 136.3 103.56) (width 0.2) (layer "B.Cu") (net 51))
 (segment (start 139.12 103.67) (end 139.09 103.64) (width 0.2) (layer "B.Cu") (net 51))
 (segment (start 133.98 99.695) (end 133.985 99.7) (width 0.2) (layer "B.Cu") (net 51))
 (segment (start 128.43 108.4) (end 128.42 108.4) (width 0.2) (layer "F.Cu") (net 54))
 (segment (start 126.43 108.4) (end 128.26 108.4) (width 0.2) (layer "F.Cu") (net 54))
 (segment (start 126.725 99.695) (end 124.3 102.12) (width 0.2) (layer "F.Cu") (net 54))
 (segment (start 132.906968 106.695001) (end 131.201969 108.4) (width 0.2) (layer "F.Cu") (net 54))
 (segment (start 124.3 102.12) (end 124.3 106.27) (width 0.2) (layer "F.Cu") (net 54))
 (segment (start 131.435001 105.394999) (end 132.906968 105.394999) (width 0.2) (layer "F.Cu") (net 54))
 (segment (start 131.201969 108.4) (end 128.42 108.4) (width 0.2) (layer "F.Cu") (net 54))
 (segment (start 124.3 106.27) (end 126.43 108.4) (width 0.2) (layer "F.Cu") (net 54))
 (segment (start 131.44 99.695) (end 132.906968 101.161968) (width 0.2) (layer "F.Cu") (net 54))
 (segment (start 128.42 108.4) (end 128.13 108.4) (width 0.2) (layer "F.Cu") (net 54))
 (segment (start 132.906968 101.161968) (end 132.906968 102.219999) (width 0.2) (layer "F.Cu") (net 54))
 (segment (start 131.435001 105.394999) (end 128.43 108.4) (width 0.2) (layer "F.Cu") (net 54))
 (segment (start 131.44 99.695) (end 126.725 99.695) (width 0.2) (layer "F.Cu") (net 54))
 (segment (start 127 102.87) (end 132.906968 102.87) (width 0.2) (layer "F.Cu") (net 52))
 (segment (start 127 105.41) (end 127 105.405) (width 0.2) (layer "F.Cu") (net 53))
 (segment (start 128.9 103.505) (end 132.891967 103.505) (width 0.2) (layer "F.Cu") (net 53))
 (segment (start 132.891967 103.505) (end 132.906968 103.520001) (width 0.2) (layer "F.Cu") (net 53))
 (segment (start 127 105.405) (end 128.9 103.505) (width 0.2) (layer "F.Cu") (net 53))
 (segment (start 139.46 99.99) (end 139.75 99.99) (width 0.2) (layer "F.Cu") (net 2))
 (segment (start 141.065 108.66136) (end 140.73636 108.99) (width 0.2) (layer "F.Cu") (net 2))
 (segment (start 137 100.96) (end 137 102.19636) (width 0.2) (layer "F.Cu") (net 2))
 (segment (start 135.063032 106.695001) (end 135.063032 107.053032) (width 0.2) (layer "F.Cu") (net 2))
 (segment (start 137 101.79636) (end 137.71864 102.515) (width 0.2) (layer "F.Cu") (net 2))
 (segment (start 137 101.57) (end 137 101.79636) (width 0.2) (layer "F.Cu") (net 2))
 (segment (start 135.063032 107.053032) (end 137 108.99) (width 0.2) (layer "F.Cu") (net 2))
 (segment (start 137 108.99) (end 140.73636 108.99) (width 0.2) (layer "F.Cu") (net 2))
 (segment (start 137.97 99.99) (end 137 100.96) (width 0.2) (layer "F.Cu") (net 2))
 (segment (start 139.465 100.76864) (end 139.465 101.265) (width 0.2) (layer "F.Cu") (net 2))
 (segment (start 140.73636 108.99) (end 145.03 108.99) (width 0.2) (layer "F.Cu") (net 2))
 (segment (start 143.065 101.265) (end 143.065 100.76864) (width 0.2) (layer "F.Cu") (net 2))
 (segment (start 146.02 108) (end 146.02 107.75) (width 0.2) (layer "F.Cu") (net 2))
 (segment (start 137.71864 102.515) (end 138.215 102.515) (width 0.2) (layer "F.Cu") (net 2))
 (segment (start 146.02 101.07) (end 144.94 99.99) (width 0.2) (layer "F.Cu") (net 2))
 (segment (start 140.34 99.99) (end 140.24364 99.99) (width 0.2) (layer "F.Cu") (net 2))
 (segment (start 146.02 108) (end 146.02 101.07) (width 0.2) (layer "F.Cu") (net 2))
 (segment (start 145.585 107.315) (end 145.115 107.315) (width 0.2) (layer "F.Cu") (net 2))
 (segment (start 139.75 99.99) (end 139.065 100.675) (width 0.2) (layer "F.Cu") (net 2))
 (segment (start 140.24364 99.99) (end 139.465 100.76864) (width 0.2) (layer "F.Cu") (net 2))
 (segment (start 145.03 108.99) (end 146.02 108) (width 0.2) (layer "F.Cu") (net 2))
 (segment (start 146.02 107.75) (end 145.585 107.315) (width 0.2) (layer "F.Cu") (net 2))
 (segment (start 137.71864 102.915) (end 138.215 102.915) (width 0.2) (layer "F.Cu") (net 2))
 (segment (start 144.94 99.99) (end 143.85 99.99) (width 0.2) (layer "F.Cu") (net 2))
 (segment (start 143.84364 99.99) (end 143.85 99.99) (width 0.2) (layer "F.Cu") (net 2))
 (segment (start 143.065 100.76864) (end 143.84364 99.99) (width 0.2) (layer "F.Cu") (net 2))
 (segment (start 137 102.19636) (end 137.71864 102.915) (width 0.2) (layer "F.Cu") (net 2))
 (segment (start 141.065 108.165) (end 141.065 108.66136) (width 0.2) (layer "F.Cu") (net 2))
 (segment (start 139.065 100.675) (end 139.065 101.265) (width 0.2) (layer "F.Cu") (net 2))
 (segment (start 143.85 99.99) (end 137.97 99.99) (width 0.2) (layer "F.Cu") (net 2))
 (segment (start 136.58 104.342046) (end 137.552954 105.315) (width 0.2) (layer "F.Cu") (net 8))
 (segment (start 135.641065 102.87) (end 136.58 103.808935) (width 0.2) (layer "F.Cu") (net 8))
 (segment (start 137.552954 105.315) (end 138.215 105.315) (width 0.2) (layer "F.Cu") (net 8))
 (segment (start 135.063032 102.87) (end 135.641065 102.87) (width 0.2) (layer "F.Cu") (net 8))
 (segment (start 136.58 103.808935) (end 136.58 104.342046) (width 0.2) (layer "F.Cu") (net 8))
 (segment (start 137.71864 104.915) (end 138.215 104.915) (width 0.2) (layer "F.Cu") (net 7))
 (segment (start 136.98 103.52) (end 136.98 104.17636) (width 0.2) (layer "F.Cu") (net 7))
 (segment (start 135.063032 102.219999) (end 135.679999 102.219999) (width 0.2) (layer "F.Cu") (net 7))
 (segment (start 135.679999 102.219999) (end 136.98 103.52) (width 0.2) (layer "F.Cu") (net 7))
 (segment (start 136.98 104.17636) (end 137.71864 104.915) (width 0.2) (layer "F.Cu") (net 7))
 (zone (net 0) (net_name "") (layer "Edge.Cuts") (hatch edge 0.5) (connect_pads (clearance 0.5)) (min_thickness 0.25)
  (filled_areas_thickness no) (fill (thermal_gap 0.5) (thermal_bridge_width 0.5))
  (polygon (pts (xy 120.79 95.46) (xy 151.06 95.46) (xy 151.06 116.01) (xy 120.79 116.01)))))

